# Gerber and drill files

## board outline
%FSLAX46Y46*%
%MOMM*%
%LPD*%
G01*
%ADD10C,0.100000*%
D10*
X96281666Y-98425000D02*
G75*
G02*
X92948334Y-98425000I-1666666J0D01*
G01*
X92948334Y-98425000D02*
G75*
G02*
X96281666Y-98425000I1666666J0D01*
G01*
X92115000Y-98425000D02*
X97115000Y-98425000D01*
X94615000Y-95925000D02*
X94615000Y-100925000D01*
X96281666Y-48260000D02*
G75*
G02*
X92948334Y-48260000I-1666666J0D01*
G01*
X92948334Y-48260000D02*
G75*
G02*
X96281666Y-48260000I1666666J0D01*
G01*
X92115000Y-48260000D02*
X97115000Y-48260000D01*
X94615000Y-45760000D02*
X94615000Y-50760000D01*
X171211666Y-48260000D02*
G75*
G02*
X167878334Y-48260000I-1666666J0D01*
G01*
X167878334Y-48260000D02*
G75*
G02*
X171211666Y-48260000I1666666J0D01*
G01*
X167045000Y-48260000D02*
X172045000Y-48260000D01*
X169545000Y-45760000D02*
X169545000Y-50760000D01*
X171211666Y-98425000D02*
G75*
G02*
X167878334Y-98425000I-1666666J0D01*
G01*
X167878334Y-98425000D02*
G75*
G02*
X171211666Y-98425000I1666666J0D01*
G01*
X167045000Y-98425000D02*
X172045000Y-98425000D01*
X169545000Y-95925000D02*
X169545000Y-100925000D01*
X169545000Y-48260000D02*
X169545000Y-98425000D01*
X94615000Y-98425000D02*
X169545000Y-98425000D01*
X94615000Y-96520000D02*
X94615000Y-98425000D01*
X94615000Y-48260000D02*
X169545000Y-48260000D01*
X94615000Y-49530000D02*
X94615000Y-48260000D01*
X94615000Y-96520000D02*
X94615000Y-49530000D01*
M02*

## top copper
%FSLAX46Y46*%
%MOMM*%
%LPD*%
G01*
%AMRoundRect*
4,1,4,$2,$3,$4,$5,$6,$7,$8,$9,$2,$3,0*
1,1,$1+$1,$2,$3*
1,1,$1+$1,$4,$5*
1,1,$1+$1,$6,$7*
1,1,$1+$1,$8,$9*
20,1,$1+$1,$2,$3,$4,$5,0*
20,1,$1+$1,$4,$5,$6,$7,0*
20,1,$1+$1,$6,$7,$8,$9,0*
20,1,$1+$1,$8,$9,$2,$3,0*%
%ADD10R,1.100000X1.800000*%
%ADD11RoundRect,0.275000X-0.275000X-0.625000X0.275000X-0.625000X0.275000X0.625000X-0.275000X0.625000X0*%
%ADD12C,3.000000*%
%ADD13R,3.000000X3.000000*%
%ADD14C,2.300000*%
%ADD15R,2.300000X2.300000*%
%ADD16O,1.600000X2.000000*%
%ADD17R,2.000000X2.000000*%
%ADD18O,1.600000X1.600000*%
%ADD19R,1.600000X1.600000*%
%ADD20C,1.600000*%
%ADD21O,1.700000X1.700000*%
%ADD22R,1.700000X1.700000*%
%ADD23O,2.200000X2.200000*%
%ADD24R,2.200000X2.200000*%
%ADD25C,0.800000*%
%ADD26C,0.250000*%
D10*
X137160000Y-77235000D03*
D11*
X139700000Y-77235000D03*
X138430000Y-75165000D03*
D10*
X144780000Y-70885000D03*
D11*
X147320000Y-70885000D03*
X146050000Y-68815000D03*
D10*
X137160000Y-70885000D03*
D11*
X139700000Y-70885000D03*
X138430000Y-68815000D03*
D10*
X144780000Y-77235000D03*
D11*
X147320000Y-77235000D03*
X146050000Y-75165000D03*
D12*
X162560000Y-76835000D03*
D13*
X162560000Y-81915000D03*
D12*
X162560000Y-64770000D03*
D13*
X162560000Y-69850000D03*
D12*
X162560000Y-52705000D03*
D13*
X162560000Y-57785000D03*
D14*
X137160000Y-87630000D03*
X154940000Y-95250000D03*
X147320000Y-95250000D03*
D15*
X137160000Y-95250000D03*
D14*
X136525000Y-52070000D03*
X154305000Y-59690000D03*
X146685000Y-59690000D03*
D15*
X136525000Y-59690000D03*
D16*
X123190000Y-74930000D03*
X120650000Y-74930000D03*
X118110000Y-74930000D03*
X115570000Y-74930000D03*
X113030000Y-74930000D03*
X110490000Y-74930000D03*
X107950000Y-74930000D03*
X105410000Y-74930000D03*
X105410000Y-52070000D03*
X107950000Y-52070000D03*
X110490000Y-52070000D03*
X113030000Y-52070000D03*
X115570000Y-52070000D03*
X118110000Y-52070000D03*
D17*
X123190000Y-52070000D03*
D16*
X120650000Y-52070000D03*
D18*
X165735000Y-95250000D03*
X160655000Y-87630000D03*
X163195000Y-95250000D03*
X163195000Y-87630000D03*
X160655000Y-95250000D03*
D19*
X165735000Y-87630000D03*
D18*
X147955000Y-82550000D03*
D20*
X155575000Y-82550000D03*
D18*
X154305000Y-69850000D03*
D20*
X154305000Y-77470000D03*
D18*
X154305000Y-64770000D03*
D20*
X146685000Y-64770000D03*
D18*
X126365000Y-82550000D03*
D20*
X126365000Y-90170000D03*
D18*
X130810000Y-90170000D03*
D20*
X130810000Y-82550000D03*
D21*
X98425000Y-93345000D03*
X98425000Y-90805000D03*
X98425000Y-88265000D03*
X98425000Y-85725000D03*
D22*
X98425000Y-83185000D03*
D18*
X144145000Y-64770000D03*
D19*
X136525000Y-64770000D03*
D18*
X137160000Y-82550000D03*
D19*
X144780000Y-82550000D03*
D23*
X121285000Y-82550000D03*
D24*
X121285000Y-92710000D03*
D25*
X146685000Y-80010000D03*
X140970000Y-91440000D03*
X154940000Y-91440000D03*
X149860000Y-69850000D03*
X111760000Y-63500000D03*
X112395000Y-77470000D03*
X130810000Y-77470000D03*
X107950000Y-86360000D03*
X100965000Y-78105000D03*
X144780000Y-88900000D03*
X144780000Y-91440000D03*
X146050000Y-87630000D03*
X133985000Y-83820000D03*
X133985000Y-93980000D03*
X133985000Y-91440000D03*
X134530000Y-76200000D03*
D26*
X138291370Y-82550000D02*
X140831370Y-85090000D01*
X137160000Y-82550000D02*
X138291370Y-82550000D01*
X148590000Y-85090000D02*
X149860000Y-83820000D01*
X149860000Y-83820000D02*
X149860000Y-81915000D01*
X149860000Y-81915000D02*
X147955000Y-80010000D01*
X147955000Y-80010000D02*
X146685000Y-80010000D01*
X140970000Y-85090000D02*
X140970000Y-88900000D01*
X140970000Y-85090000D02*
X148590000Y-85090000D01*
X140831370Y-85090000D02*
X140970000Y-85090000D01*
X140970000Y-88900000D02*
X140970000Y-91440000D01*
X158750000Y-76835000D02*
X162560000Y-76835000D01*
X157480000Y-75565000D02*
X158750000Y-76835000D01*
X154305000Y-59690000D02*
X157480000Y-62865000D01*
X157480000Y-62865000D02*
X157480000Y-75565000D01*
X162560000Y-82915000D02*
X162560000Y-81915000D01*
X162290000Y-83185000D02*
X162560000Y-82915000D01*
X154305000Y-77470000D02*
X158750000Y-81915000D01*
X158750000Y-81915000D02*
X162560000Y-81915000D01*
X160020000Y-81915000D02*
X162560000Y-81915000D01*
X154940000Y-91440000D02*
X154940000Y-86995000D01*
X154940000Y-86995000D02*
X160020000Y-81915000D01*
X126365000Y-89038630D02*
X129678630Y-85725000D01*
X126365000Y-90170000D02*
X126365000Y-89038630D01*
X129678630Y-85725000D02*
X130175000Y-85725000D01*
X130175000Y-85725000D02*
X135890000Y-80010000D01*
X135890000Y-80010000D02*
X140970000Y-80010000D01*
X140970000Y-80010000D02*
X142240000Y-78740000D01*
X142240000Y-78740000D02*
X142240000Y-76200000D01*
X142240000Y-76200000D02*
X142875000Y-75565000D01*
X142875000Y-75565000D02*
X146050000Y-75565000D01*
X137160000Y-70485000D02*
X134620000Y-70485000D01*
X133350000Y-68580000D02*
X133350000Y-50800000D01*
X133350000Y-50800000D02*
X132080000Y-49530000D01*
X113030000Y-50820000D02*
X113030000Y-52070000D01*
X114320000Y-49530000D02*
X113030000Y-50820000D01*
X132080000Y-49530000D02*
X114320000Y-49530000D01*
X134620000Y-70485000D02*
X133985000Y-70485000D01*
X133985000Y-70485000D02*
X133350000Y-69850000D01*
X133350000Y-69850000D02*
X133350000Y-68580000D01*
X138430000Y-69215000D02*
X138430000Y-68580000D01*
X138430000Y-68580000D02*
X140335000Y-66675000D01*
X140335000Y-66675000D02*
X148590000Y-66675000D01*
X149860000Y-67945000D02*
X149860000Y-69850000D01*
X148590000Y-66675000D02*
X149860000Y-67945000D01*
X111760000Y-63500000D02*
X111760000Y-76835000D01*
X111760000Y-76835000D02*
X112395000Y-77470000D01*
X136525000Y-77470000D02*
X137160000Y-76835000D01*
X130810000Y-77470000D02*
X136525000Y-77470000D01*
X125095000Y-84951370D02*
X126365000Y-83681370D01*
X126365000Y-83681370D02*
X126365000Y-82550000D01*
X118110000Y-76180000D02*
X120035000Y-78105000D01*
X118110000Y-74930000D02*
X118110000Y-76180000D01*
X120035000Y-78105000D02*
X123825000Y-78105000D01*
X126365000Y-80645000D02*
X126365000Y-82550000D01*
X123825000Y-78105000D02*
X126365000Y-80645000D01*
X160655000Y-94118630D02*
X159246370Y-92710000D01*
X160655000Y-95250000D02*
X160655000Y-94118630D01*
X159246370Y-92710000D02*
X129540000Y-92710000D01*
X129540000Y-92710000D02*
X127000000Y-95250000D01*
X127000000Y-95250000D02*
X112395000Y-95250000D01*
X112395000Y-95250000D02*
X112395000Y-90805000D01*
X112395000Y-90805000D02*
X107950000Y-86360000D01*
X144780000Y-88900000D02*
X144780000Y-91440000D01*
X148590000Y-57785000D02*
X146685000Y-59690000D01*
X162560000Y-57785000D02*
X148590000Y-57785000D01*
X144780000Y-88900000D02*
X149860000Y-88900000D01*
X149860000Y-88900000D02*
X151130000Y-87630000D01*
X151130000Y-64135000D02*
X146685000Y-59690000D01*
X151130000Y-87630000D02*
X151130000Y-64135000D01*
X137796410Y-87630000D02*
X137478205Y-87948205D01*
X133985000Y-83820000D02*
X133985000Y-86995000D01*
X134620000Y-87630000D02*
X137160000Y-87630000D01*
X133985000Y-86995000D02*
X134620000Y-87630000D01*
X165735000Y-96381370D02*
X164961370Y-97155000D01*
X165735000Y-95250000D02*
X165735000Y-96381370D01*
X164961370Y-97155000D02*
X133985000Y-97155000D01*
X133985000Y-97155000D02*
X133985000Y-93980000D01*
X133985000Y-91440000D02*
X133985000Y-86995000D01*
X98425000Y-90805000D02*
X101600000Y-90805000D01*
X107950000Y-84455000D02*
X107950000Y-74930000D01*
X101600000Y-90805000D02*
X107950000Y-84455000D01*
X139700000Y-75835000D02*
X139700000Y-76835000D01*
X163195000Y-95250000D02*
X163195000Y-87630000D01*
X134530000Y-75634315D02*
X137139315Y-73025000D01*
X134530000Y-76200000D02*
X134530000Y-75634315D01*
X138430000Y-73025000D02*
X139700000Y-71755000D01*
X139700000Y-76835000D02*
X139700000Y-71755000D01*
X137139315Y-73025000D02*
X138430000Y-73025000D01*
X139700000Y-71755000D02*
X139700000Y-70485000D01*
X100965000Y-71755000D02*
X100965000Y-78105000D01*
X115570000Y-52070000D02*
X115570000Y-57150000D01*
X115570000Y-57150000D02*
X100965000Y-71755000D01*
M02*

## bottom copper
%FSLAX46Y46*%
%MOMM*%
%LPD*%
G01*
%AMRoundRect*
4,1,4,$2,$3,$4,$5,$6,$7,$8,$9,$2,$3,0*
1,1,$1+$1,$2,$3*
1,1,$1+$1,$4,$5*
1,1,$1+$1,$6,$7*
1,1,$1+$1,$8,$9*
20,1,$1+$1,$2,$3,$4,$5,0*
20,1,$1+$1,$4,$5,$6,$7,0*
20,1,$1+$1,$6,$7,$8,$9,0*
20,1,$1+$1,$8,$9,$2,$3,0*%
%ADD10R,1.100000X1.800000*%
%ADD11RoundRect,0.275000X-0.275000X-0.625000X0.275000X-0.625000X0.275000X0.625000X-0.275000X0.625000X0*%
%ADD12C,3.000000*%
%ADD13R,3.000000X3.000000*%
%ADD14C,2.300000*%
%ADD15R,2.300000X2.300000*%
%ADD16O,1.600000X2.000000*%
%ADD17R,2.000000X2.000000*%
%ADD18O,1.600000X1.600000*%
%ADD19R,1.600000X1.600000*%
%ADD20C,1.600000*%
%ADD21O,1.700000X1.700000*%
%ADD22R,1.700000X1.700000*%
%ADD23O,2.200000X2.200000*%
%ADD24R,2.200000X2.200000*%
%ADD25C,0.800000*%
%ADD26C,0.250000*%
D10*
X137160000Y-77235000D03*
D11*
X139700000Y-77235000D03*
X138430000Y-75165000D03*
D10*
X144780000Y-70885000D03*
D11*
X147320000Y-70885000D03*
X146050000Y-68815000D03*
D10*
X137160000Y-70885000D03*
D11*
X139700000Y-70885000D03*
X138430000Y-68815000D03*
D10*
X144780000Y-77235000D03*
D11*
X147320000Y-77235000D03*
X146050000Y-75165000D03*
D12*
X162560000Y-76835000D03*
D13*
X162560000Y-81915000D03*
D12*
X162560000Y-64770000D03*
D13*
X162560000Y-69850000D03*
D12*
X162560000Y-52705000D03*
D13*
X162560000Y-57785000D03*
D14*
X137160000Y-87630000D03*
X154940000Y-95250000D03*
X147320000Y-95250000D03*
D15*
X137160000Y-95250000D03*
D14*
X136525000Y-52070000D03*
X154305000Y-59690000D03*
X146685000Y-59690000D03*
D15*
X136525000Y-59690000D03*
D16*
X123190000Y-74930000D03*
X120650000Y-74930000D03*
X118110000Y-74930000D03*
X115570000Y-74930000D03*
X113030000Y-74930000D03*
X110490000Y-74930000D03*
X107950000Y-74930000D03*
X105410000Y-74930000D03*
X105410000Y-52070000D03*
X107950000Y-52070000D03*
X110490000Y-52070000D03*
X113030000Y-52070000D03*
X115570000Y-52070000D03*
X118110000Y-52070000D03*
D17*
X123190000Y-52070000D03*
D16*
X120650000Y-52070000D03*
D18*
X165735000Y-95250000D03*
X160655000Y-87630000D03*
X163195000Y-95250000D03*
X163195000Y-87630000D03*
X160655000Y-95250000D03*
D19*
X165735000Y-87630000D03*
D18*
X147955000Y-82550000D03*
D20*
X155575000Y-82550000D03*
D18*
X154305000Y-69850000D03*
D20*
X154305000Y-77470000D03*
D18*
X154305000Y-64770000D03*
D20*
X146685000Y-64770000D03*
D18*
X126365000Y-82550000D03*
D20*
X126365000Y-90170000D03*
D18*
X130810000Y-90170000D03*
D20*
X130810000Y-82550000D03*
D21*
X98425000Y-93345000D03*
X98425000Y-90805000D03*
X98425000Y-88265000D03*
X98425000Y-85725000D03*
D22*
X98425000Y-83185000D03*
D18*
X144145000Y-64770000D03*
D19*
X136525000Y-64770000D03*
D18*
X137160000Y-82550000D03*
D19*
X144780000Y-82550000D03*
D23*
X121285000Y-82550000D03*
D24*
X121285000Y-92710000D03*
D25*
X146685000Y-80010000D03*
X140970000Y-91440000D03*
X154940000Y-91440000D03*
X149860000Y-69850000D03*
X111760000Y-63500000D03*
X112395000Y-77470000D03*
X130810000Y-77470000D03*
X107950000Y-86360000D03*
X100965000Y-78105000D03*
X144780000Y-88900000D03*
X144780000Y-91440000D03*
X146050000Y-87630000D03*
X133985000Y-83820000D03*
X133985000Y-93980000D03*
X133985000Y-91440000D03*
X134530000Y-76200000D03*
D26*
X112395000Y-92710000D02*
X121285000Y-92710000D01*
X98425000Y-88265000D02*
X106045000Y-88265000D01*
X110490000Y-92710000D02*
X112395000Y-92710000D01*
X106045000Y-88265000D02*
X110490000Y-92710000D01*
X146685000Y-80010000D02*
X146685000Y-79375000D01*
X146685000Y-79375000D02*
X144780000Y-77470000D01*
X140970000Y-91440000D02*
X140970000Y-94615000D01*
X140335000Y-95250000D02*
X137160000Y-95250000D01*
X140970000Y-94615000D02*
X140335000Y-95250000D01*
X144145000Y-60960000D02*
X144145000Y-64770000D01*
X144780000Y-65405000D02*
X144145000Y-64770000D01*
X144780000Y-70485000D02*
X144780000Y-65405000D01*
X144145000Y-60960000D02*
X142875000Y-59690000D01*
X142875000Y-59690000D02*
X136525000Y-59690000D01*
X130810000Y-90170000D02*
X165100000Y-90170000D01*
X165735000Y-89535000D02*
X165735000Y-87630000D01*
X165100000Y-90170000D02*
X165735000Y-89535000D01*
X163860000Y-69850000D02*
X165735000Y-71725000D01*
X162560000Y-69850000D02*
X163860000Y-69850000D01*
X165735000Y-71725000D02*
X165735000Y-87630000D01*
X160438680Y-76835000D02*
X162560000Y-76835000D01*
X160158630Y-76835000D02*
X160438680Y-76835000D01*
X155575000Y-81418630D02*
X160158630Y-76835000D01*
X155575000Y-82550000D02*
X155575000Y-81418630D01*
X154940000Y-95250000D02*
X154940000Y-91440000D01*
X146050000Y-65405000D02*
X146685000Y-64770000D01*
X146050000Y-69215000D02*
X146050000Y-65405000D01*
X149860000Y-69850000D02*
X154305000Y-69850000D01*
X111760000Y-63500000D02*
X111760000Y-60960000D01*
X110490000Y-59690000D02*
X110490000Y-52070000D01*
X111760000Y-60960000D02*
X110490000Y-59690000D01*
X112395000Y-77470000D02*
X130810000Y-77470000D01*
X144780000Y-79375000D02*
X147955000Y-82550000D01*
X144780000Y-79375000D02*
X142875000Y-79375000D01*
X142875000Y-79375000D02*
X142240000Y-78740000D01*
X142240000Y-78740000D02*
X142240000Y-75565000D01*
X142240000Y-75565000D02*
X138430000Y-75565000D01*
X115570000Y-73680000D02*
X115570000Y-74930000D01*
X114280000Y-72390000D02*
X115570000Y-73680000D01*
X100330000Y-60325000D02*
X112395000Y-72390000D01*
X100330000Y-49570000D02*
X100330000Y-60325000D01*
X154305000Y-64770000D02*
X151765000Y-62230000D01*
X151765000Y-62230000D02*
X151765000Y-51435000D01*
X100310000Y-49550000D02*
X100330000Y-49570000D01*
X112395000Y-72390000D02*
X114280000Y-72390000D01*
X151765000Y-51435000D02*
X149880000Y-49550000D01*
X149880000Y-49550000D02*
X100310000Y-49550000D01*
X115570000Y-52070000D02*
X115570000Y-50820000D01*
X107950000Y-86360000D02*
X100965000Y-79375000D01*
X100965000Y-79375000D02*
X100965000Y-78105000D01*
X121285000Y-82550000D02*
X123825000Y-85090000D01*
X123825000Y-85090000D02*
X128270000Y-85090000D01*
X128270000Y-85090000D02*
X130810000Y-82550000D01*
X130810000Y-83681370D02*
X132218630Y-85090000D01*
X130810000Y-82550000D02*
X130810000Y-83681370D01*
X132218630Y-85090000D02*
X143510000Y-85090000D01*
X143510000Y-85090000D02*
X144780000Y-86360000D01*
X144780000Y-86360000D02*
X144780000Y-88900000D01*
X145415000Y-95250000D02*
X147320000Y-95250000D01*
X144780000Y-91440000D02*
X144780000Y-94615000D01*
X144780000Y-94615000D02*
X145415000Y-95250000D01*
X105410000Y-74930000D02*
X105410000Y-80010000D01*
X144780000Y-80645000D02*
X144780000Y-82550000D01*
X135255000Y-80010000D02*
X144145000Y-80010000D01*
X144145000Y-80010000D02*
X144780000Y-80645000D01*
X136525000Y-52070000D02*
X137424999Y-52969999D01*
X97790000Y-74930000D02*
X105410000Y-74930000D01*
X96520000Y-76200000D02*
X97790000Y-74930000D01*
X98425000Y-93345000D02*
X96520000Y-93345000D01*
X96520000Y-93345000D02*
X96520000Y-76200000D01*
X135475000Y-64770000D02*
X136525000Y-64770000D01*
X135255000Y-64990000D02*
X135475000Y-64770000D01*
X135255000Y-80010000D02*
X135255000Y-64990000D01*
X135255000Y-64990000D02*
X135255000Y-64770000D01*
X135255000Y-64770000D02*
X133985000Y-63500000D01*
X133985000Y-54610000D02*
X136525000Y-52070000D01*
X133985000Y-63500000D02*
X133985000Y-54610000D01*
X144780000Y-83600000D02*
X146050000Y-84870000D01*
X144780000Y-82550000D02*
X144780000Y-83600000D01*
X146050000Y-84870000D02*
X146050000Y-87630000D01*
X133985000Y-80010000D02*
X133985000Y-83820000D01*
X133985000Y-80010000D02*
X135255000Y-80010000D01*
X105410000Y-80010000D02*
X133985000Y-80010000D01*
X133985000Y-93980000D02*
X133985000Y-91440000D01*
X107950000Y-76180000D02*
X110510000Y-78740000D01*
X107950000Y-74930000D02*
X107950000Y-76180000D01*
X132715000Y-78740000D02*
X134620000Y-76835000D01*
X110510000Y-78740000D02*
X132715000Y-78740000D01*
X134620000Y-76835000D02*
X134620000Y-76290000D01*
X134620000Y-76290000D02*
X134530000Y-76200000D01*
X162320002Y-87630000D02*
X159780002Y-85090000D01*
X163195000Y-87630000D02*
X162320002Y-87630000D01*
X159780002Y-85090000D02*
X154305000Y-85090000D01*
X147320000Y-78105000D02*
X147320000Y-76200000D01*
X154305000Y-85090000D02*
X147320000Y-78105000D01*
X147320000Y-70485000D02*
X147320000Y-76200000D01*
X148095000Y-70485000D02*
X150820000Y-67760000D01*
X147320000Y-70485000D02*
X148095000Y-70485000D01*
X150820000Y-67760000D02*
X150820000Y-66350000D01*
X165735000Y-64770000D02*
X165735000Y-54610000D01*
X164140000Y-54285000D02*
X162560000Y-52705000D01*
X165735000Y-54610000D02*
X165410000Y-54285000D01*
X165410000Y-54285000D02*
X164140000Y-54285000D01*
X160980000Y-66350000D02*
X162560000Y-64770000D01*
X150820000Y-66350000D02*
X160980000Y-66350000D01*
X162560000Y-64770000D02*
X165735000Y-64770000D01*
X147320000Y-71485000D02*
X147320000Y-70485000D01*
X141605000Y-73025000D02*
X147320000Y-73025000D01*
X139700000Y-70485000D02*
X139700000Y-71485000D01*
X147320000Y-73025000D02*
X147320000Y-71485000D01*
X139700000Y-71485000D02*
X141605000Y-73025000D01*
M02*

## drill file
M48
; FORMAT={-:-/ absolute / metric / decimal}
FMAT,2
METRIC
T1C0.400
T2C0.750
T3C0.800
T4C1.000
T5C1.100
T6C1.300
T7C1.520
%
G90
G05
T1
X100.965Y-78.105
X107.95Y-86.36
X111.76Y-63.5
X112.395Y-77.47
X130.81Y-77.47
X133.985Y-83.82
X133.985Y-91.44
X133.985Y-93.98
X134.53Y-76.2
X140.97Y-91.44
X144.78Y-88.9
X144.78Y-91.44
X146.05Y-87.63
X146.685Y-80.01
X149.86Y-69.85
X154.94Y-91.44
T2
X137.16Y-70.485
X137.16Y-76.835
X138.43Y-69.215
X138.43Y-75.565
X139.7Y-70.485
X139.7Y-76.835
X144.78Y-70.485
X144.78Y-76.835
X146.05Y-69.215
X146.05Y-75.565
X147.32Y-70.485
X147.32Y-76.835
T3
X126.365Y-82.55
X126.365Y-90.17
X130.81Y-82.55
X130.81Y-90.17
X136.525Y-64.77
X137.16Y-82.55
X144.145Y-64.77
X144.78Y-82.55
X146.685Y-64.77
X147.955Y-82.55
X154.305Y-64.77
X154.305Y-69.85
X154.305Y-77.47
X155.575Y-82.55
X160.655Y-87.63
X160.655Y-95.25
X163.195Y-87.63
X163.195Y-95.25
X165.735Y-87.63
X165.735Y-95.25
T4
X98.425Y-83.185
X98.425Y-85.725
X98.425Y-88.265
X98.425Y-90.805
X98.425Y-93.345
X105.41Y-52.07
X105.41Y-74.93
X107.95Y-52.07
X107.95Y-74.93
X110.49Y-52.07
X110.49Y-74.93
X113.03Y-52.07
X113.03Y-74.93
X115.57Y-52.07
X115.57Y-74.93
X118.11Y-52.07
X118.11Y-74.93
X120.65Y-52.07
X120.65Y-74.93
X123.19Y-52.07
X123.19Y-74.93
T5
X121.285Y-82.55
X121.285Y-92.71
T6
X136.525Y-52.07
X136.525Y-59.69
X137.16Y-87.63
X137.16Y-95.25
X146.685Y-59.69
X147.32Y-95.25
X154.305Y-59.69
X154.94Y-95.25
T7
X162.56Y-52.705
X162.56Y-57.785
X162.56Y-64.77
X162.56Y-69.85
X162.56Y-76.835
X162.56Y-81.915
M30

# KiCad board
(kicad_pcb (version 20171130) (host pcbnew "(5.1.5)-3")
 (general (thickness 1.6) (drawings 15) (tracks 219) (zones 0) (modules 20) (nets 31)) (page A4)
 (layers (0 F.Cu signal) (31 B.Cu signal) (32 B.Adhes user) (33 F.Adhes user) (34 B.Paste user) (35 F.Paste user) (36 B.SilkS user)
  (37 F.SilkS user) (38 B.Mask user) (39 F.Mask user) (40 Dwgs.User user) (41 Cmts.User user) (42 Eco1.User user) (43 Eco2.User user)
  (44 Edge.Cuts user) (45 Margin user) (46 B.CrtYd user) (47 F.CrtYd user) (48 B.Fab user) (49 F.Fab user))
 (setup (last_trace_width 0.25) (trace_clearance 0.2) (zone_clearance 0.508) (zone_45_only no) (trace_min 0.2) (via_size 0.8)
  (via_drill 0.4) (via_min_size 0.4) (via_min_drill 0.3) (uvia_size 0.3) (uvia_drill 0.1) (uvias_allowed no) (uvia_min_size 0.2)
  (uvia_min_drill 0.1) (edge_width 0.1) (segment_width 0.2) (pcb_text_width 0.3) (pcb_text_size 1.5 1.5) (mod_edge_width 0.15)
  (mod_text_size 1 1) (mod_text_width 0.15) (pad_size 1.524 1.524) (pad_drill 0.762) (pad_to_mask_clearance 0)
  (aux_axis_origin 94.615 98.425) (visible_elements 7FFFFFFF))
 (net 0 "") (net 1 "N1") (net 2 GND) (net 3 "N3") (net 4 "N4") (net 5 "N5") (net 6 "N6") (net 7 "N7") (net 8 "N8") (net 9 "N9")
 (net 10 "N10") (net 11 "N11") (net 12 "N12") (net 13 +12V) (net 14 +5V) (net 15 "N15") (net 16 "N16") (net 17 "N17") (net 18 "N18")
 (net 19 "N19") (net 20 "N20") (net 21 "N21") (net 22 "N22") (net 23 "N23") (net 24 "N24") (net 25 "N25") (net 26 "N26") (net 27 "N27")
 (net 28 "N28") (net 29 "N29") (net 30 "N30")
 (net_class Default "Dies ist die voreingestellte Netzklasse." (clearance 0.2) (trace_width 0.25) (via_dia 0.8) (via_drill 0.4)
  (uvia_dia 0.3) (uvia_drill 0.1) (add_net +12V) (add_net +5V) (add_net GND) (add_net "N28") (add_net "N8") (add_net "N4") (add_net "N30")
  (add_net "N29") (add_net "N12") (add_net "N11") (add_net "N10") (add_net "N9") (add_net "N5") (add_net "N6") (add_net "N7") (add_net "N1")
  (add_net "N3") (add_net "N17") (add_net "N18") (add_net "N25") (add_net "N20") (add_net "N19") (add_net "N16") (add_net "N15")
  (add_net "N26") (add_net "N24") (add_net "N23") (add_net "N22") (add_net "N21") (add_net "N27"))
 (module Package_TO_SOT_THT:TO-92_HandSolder (layer F.Cu) (at 137.16 76.835)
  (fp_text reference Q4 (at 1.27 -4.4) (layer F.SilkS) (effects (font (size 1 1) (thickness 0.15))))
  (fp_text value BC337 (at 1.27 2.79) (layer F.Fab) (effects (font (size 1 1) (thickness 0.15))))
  (pad 1 thru_hole rect (at 0 0) (size 1.1 1.8) (drill 0.75 (offset 0 0.4)) (layers *.Cu *.Mask) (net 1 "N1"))
  (pad 3 thru_hole roundrect (at 2.54 0) (size 1.1 1.8) (drill 0.75 (offset 0 0.4)) (layers *.Cu *.Mask) (roundrect_rratio 0.25) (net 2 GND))
  (pad 2 thru_hole roundrect (at 1.27 -1.27) (size 1.1 1.8) (drill 0.75 (offset 0 -0.4)) (layers *.Cu *.Mask) (roundrect_rratio 0.25)
   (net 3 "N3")))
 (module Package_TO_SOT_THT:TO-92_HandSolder (layer F.Cu) (at 144.78 70.485)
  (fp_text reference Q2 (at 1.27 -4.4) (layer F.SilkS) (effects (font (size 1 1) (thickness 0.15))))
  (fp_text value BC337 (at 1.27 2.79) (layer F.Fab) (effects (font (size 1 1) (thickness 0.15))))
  (pad 1 thru_hole rect (at 0 0) (size 1.1 1.8) (drill 0.75 (offset 0 0.4)) (layers *.Cu *.Mask) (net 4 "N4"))
  (pad 3 thru_hole roundrect (at 2.54 0) (size 1.1 1.8) (drill 0.75 (offset 0 0.4)) (layers *.Cu *.Mask) (roundrect_rratio 0.25) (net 2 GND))
  (pad 2 thru_hole roundrect (at 1.27 -1.27) (size 1.1 1.8) (drill 0.75 (offset 0 -0.4)) (layers *.Cu *.Mask) (roundrect_rratio 0.25)
   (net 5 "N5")))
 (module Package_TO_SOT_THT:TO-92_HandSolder (layer F.Cu) (at 137.16 70.485)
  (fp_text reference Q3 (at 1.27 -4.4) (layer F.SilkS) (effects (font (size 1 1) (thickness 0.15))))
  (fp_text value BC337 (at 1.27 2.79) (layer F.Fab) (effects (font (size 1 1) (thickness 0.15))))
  (pad 1 thru_hole rect (at 0 0) (size 1.1 1.8) (drill 0.75 (offset 0 0.4)) (layers *.Cu *.Mask) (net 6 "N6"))
  (pad 3 thru_hole roundrect (at 2.54 0) (size 1.1 1.8) (drill 0.75 (offset 0 0.4)) (layers *.Cu *.Mask) (roundrect_rratio 0.25) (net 2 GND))
  (pad 2 thru_hole roundrect (at 1.27 -1.27) (size 1.1 1.8) (drill 0.75 (offset 0 -0.4)) (layers *.Cu *.Mask) (roundrect_rratio 0.25)
   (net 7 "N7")))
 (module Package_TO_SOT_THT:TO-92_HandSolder (layer F.Cu) (at 144.78 76.835)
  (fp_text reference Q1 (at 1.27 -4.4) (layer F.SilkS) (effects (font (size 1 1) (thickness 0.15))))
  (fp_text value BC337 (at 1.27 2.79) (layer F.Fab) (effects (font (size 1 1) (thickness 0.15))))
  (pad 1 thru_hole rect (at 0 0) (size 1.1 1.8) (drill 0.75 (offset 0 0.4)) (layers *.Cu *.Mask) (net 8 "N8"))
  (pad 3 thru_hole roundrect (at 2.54 0) (size 1.1 1.8) (drill 0.75 (offset 0 0.4)) (layers *.Cu *.Mask) (roundrect_rratio 0.25) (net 2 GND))
  (pad 2 thru_hole roundrect (at 1.27 -1.27) (size 1.1 1.8) (drill 0.75 (offset 0 -0.4)) (layers *.Cu *.Mask) (roundrect_rratio 0.25)
   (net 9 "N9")))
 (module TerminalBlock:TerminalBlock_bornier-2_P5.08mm (layer F.Cu) (at 162.56 81.915 90)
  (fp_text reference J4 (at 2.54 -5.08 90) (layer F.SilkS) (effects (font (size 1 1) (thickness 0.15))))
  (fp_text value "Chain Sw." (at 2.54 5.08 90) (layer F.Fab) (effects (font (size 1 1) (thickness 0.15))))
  (pad 2 thru_hole circle (at 5.08 0 90) (size 3 3) (drill 1.52) (layers *.Cu *.Mask) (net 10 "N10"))
  (pad 1 thru_hole rect (at 0 0 90) (size 3 3) (drill 1.52) (layers *.Cu *.Mask) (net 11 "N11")))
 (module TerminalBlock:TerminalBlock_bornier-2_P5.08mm (layer F.Cu) (at 162.56 69.85 90)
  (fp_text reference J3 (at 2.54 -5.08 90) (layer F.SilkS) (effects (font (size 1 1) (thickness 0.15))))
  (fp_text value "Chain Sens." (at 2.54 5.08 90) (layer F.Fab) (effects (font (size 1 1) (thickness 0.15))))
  (pad 2 thru_hole circle (at 5.08 0 90) (size 3 3) (drill 1.52) (layers *.Cu *.Mask) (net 2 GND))
  (pad 1 thru_hole rect (at 0 0 90) (size 3 3) (drill 1.52) (layers *.Cu *.Mask) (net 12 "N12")))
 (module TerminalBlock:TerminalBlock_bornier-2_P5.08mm (layer F.Cu) (at 162.56 57.785 90)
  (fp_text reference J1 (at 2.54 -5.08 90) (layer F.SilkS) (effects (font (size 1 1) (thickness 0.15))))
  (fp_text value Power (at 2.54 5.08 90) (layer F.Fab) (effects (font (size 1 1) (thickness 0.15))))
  (pad 2 thru_hole circle (at 5.08 0 90) (size 3 3) (drill 1.52) (layers *.Cu *.Mask) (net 2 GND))
  (pad 1 thru_hole rect (at 0 0 90) (size 3 3) (drill 1.52) (layers *.Cu *.Mask) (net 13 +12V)))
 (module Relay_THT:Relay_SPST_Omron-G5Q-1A (layer F.Cu) (at 137.16 95.25)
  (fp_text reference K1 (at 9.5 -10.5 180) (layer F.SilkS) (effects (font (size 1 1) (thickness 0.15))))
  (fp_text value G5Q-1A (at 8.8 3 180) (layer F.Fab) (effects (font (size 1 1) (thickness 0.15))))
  (pad 5 thru_hole circle (at 0 -7.62 180) (size 2.3 2.3) (drill 1.3) (layers *.Cu *.Mask) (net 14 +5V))
  (pad 3 thru_hole circle (at 17.78 0 180) (size 2.3 2.3) (drill 1.3) (layers *.Cu *.Mask) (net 11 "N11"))
  (pad 2 thru_hole circle (at 10.16 0 180) (size 2.3 2.3) (drill 1.3) (layers *.Cu *.Mask) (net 13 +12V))
  (pad 1 thru_hole rect (at 0 0 180) (size 2.3 2.3) (drill 1.3) (layers *.Cu *.Mask) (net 8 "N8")))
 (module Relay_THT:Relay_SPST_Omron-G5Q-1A (layer F.Cu) (at 136.525 59.69)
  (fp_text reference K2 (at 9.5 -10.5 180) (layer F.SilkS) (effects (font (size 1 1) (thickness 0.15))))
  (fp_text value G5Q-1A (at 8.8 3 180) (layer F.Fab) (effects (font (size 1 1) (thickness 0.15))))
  (pad 5 thru_hole circle (at 0 -7.62 180) (size 2.3 2.3) (drill 1.3) (layers *.Cu *.Mask) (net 14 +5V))
  (pad 3 thru_hole circle (at 17.78 0 180) (size 2.3 2.3) (drill 1.3) (layers *.Cu *.Mask) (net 10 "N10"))
  (pad 2 thru_hole circle (at 10.16 0 180) (size 2.3 2.3) (drill 1.3) (layers *.Cu *.Mask) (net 13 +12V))
  (pad 1 thru_hole rect (at 0 0 180) (size 2.3 2.3) (drill 1.3) (layers *.Cu *.Mask) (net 4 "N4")))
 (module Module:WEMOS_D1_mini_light (layer F.Cu) (at 123.19 52.07 270)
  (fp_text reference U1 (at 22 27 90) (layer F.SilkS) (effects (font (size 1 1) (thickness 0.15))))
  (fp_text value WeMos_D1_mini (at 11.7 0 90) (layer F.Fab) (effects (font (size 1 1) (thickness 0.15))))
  (pad 16 thru_hole oval (at 22.86 0 270) (size 2 1.6) (drill 1) (layers *.Cu *.Mask) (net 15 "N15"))
  (pad 15 thru_hole oval (at 22.86 2.54 270) (size 2 1.6) (drill 1) (layers *.Cu *.Mask) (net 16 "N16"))
  (pad 14 thru_hole oval (at 22.86 5.08 270) (size 2 1.6) (drill 1) (layers *.Cu *.Mask) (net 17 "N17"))
  (pad 13 thru_hole oval (at 22.86 7.62 270) (size 2 1.6) (drill 1) (layers *.Cu *.Mask) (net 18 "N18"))
  (pad 12 thru_hole oval (at 22.86 10.16 270) (size 2 1.6) (drill 1) (layers *.Cu *.Mask) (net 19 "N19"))
  (pad 11 thru_hole oval (at 22.86 12.7 270) (size 2 1.6) (drill 1) (layers *.Cu *.Mask) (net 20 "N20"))
  (pad 10 thru_hole oval (at 22.86 15.24 270) (size 2 1.6) (drill 1) (layers *.Cu *.Mask) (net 2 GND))
  (pad 9 thru_hole oval (at 22.86 17.78 270) (size 2 1.6) (drill 1) (layers *.Cu *.Mask) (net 14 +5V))
  (pad 8 thru_hole oval (at 0 17.78 270) (size 2 1.6) (drill 1) (layers *.Cu *.Mask) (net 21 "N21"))
  (pad 7 thru_hole oval (at 0 15.24 270) (size 2 1.6) (drill 1) (layers *.Cu *.Mask) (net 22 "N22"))
  (pad 6 thru_hole oval (at 0 12.7 270) (size 2 1.6) (drill 1) (layers *.Cu *.Mask) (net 1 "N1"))
  (pad 5 thru_hole oval (at 0 10.16 270) (size 2 1.6) (drill 1) (layers *.Cu *.Mask) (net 6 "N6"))
  (pad 4 thru_hole oval (at 0 7.62 270) (size 2 1.6) (drill 1) (layers *.Cu *.Mask) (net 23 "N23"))
  (pad 3 thru_hole oval (at 0 5.08 270) (size 2 1.6) (drill 1) (layers *.Cu *.Mask) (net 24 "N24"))
  (pad 1 thru_hole rect (at 0 0 270) (size 2 2) (drill 1) (layers *.Cu *.Mask) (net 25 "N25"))
  (pad 2 thru_hole oval (at 0 2.54 270) (size 2 1.6) (drill 1) (layers *.Cu *.Mask) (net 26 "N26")))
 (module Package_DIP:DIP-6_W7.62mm (layer F.Cu) (at 165.735 87.63 270)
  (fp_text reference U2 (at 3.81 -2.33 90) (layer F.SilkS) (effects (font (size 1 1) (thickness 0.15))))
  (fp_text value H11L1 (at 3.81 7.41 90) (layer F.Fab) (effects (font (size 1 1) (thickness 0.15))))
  (pad 6 thru_hole oval (at 7.62 0 270) (size 1.6 1.6) (drill 0.8) (layers *.Cu *.Mask) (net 14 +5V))
  (pad 3 thru_hole oval (at 0 5.08 270) (size 1.6 1.6) (drill 0.8) (layers *.Cu *.Mask) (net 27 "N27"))
  (pad 5 thru_hole oval (at 7.62 2.54 270) (size 1.6 1.6) (drill 0.8) (layers *.Cu *.Mask) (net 2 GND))
  (pad 2 thru_hole oval (at 0 2.54 270) (size 1.6 1.6) (drill 0.8) (layers *.Cu *.Mask) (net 2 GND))
  (pad 4 thru_hole oval (at 7.62 5.08 270) (size 1.6 1.6) (drill 0.8) (layers *.Cu *.Mask) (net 23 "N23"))
  (pad 1 thru_hole rect (at 0 0 270) (size 1.6 1.6) (drill 0.8) (layers *.Cu *.Mask) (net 12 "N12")))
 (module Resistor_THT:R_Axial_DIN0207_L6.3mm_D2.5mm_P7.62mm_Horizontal (layer F.Cu) (at 155.575 82.55 180)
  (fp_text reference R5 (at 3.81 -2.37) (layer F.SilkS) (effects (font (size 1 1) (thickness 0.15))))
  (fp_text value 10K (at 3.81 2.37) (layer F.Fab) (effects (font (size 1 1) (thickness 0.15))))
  (pad 2 thru_hole oval (at 7.62 0 180) (size 1.6 1.6) (drill 0.8) (layers *.Cu *.Mask) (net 3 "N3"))
  (pad 1 thru_hole circle (at 0 0 180) (size 1.6 1.6) (drill 0.8) (layers *.Cu *.Mask) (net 10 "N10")))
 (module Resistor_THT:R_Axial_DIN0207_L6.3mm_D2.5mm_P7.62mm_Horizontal (layer F.Cu) (at 154.305 77.47 90)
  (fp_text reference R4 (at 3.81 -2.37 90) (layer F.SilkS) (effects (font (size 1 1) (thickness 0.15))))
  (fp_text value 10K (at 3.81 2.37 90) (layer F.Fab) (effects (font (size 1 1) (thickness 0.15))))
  (pad 2 thru_hole oval (at 7.62 0 90) (size 1.6 1.6) (drill 0.8) (layers *.Cu *.Mask) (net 7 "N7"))
  (pad 1 thru_hole circle (at 0 0 90) (size 1.6 1.6) (drill 0.8) (layers *.Cu *.Mask) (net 11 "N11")))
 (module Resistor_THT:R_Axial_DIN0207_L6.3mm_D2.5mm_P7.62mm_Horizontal (layer F.Cu) (at 146.685 64.77)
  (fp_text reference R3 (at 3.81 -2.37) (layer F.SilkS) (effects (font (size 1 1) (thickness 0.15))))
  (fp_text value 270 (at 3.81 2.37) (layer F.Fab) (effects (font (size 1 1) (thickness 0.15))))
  (pad 2 thru_hole oval (at 7.62 0) (size 1.6 1.6) (drill 0.8) (layers *.Cu *.Mask) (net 18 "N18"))
  (pad 1 thru_hole circle (at 0 0) (size 1.6 1.6) (drill 0.8) (layers *.Cu *.Mask) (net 5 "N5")))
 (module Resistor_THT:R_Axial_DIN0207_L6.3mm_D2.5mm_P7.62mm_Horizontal (layer F.Cu) (at 126.365 90.17 90)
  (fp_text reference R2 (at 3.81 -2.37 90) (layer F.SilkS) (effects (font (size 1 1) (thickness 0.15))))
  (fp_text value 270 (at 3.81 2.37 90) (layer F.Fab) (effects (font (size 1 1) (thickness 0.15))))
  (pad 2 thru_hole oval (at 7.62 0 90) (size 1.6 1.6) (drill 0.8) (layers *.Cu *.Mask) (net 17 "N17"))
  (pad 1 thru_hole circle (at 0 0 90) (size 1.6 1.6) (drill 0.8) (layers *.Cu *.Mask) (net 9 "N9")))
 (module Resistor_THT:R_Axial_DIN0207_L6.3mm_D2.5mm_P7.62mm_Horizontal (layer F.Cu) (at 130.81 82.55 270)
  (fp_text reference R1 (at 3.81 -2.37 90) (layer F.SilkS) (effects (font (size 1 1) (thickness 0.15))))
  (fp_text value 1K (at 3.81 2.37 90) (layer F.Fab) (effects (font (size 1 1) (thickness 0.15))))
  (pad 2 thru_hole oval (at 7.62 0 270) (size 1.6 1.6) (drill 0.8) (layers *.Cu *.Mask) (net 12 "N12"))
  (pad 1 thru_hole circle (at 0 0 270) (size 1.6 1.6) (drill 0.8) (layers *.Cu *.Mask) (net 13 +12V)))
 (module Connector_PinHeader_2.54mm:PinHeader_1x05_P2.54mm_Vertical (layer F.Cu) (at 98.425 83.185)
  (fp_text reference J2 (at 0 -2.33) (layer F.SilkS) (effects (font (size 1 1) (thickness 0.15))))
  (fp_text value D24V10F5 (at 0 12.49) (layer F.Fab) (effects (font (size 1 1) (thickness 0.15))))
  (pad 5 thru_hole oval (at 0 10.16) (size 1.7 1.7) (drill 1) (layers *.Cu *.Mask) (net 14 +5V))
  (pad 4 thru_hole oval (at 0 7.62) (size 1.7 1.7) (drill 1) (layers *.Cu *.Mask) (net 2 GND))
  (pad 3 thru_hole oval (at 0 5.08) (size 1.7 1.7) (drill 1) (layers *.Cu *.Mask) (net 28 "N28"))
  (pad 2 thru_hole oval (at 0 2.54) (size 1.7 1.7) (drill 1) (layers *.Cu *.Mask) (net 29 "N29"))
  (pad 1 thru_hole rect (at 0 0) (size 1.7 1.7) (drill 1) (layers *.Cu *.Mask) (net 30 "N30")))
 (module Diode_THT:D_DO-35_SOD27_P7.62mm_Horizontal (layer F.Cu) (at 136.525 64.77)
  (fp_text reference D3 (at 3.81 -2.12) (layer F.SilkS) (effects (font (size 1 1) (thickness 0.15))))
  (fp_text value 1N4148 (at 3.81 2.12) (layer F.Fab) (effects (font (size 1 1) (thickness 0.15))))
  (pad 2 thru_hole oval (at 7.62 0) (size 1.6 1.6) (drill 0.8) (layers *.Cu *.Mask) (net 4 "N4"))
  (pad 1 thru_hole rect (at 0 0) (size 1.6 1.6) (drill 0.8) (layers *.Cu *.Mask) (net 14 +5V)))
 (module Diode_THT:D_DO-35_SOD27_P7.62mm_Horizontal (layer F.Cu) (at 144.78 82.55 180)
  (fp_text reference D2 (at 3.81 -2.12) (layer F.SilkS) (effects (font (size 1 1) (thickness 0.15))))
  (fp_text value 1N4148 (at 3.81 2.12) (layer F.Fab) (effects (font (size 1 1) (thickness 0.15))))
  (pad 2 thru_hole oval (at 7.62 0 180) (size 1.6 1.6) (drill 0.8) (layers *.Cu *.Mask) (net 8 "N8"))
  (pad 1 thru_hole rect (at 0 0 180) (size 1.6 1.6) (drill 0.8) (layers *.Cu *.Mask) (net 14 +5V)))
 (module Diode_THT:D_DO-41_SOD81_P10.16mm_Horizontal (layer F.Cu) (at 121.285 92.71 90)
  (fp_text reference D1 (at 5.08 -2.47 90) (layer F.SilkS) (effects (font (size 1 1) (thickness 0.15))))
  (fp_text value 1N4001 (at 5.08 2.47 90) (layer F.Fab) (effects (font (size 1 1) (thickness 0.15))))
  (pad 2 thru_hole oval (at 10.16 0 90) (size 2.2 2.2) (drill 1.1) (layers *.Cu *.Mask) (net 13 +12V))
  (pad 1 thru_hole rect (at 0 0 90) (size 2.2 2.2) (drill 1.1) (layers *.Cu *.Mask) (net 28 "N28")))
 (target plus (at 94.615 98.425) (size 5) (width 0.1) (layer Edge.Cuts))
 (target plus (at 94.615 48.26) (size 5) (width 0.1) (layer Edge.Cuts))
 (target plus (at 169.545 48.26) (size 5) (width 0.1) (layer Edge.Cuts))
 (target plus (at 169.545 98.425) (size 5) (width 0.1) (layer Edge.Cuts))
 (gr_line (start 169.545 48.26) (end 169.545 98.425) (layer Edge.Cuts) (width 0.1))
 (gr_line (start 94.615 98.425) (end 169.545 98.425) (layer Edge.Cuts) (width 0.1))
 (gr_line (start 94.615 96.52) (end 94.615 98.425) (layer Edge.Cuts) (width 0.1))
 (gr_line (start 94.615 48.26) (end 169.545 48.26) (layer Edge.Cuts) (width 0.1))
 (gr_line (start 94.615 49.53) (end 94.615 48.26) (layer Edge.Cuts) (width 0.1))
 (gr_line (start 94.615 96.52) (end 94.615 49.53) (layer Edge.Cuts) (width 0.1))
 (segment (start 112.395 92.71) (end 121.285 92.71) (width 0.25) (layer B.Cu) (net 28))
 (segment (start 98.425 88.265) (end 106.045 88.265) (width 0.25) (layer B.Cu) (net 28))
 (segment (start 110.49 92.71) (end 112.395 92.71) (width 0.25) (layer B.Cu) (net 28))
 (segment (start 106.045 88.265) (end 110.49 92.71) (width 0.25) (layer B.Cu) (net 28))
 (segment (start 138.29137 82.55) (end 140.83137 85.09) (width 0.25) (layer F.Cu) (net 8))
 (segment (start 137.16 82.55) (end 138.29137 82.55) (width 0.25) (layer F.Cu) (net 8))
 (segment (start 148.59 85.09) (end 149.86 83.82) (width 0.25) (layer F.Cu) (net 8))
 (segment (start 149.86 83.82) (end 149.86 81.915) (width 0.25) (layer F.Cu) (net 8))
 (segment (start 149.86 81.915) (end 147.955 80.01) (width 0.25) (layer F.Cu) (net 8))
 (via (at 146.685 80.01) (size 0.8) (drill 0.4) (layers F.Cu B.Cu) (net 8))
 (segment (start 147.955 80.01) (end 146.685 80.01) (width 0.25) (layer F.Cu) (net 8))
 (segment (start 146.685 80.01) (end 146.685 79.375) (width 0.25) (layer B.Cu) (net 8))
 (segment (start 146.685 79.375) (end 144.78 77.47) (width 0.25) (layer B.Cu) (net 8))
 (segment (start 140.97 85.09) (end 140.97 88.9) (width 0.25) (layer F.Cu) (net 8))
 (segment (start 140.97 85.09) (end 148.59 85.09) (width 0.25) (layer F.Cu) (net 8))
 (segment (start 140.83137 85.09) (end 140.97 85.09) (width 0.25) (layer F.Cu) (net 8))
 (segment (start 140.97 88.9) (end 140.97 91.44) (width 0.25) (layer F.Cu) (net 8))
 (via (at 140.97 91.44) (size 0.8) (drill 0.4) (layers F.Cu B.Cu) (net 8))
 (segment (start 140.97 91.44) (end 140.97 94.615) (width 0.25) (layer B.Cu) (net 8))
 (segment (start 140.335 95.25) (end 137.16 95.25) (width 0.25) (layer B.Cu) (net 8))
 (segment (start 140.97 94.615) (end 140.335 95.25) (width 0.25) (layer B.Cu) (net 8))
 (segment (start 144.145 60.96) (end 144.145 64.77) (width 0.25) (layer B.Cu) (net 4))
 (segment (start 144.78 65.405) (end 144.145 64.77) (width 0.25) (layer B.Cu) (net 4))
 (segment (start 144.78 70.485) (end 144.78 65.405) (width 0.25) (layer B.Cu) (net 4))
 (segment (start 144.145 60.96) (end 142.875 59.69) (width 0.25) (layer B.Cu) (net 4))
 (segment (start 142.875 59.69) (end 136.525 59.69) (width 0.25) (layer B.Cu) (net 4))
 (segment (start 130.81 90.17) (end 165.1 90.17) (width 0.25) (layer B.Cu) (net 12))
 (segment (start 165.735 89.535) (end 165.735 87.63) (width 0.25) (layer B.Cu) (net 12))
 (segment (start 165.1 90.17) (end 165.735 89.535) (width 0.25) (layer B.Cu) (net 12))
 (segment (start 163.86 69.85) (end 165.735 71.725) (width 0.25) (layer B.Cu) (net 12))
 (segment (start 162.56 69.85) (end 163.86 69.85) (width 0.25) (layer B.Cu) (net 12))
 (segment (start 165.735 71.725) (end 165.735 87.63) (width 0.25) (layer B.Cu) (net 12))
 (segment (start 158.75 76.835) (end 162.56 76.835) (width 0.25) (layer F.Cu) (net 10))
 (segment (start 157.48 75.565) (end 158.75 76.835) (width 0.25) (layer F.Cu) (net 10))
 (segment (start 154.305 59.69) (end 157.48 62.865) (width 0.25) (layer F.Cu) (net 10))
 (segment (start 157.48 62.865) (end 157.48 75.565) (width 0.25) (layer F.Cu) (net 10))
 (segment (start 160.43868 76.835) (end 162.56 76.835) (width 0.25) (layer B.Cu) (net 10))
 (segment (start 160.15863 76.835) (end 160.43868 76.835) (width 0.25) (layer B.Cu) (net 10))
 (segment (start 155.575 81.41863) (end 160.15863 76.835) (width 0.25) (layer B.Cu) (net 10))
 (segment (start 155.575 82.55) (end 155.575 81.41863) (width 0.25) (layer B.Cu) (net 10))
 (segment (start 154.94 95.25) (end 154.94 91.44) (width 0.25) (layer B.Cu) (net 11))
 (via (at 154.94 91.44) (size 0.8) (drill 0.4) (layers F.Cu B.Cu) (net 11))
 (segment (start 162.56 82.915) (end 162.56 81.915) (width 0.25) (layer F.Cu) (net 11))
 (segment (start 162.29 83.185) (end 162.56 82.915) (width 0.25) (layer F.Cu) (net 11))
 (segment (start 154.305 77.47) (end 158.75 81.915) (width 0.25) (layer F.Cu) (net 11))
 (segment (start 158.75 81.915) (end 162.56 81.915) (width 0.25) (layer F.Cu) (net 11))
 (segment (start 160.02 81.915) (end 162.56 81.915) (width 0.25) (layer F.Cu) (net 11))
 (segment (start 154.94 91.44) (end 154.94 86.995) (width 0.25) (layer F.Cu) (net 11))
 (segment (start 154.94 86.995) (end 160.02 81.915) (width 0.25) (layer F.Cu) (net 11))
 (segment (start 126.365 89.03863) (end 129.67863 85.725) (width 0.25) (layer F.Cu) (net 9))
 (segment (start 126.365 90.17) (end 126.365 89.03863) (width 0.25) (layer F.Cu) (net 9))
 (segment (start 129.67863 85.725) (end 130.175 85.725) (width 0.25) (layer F.Cu) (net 9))
 (segment (start 130.175 85.725) (end 135.89 80.01) (width 0.25) (layer F.Cu) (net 9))
 (segment (start 135.89 80.01) (end 140.97 80.01) (width 0.25) (layer F.Cu) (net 9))
 (segment (start 140.97 80.01) (end 142.24 78.74) (width 0.25) (layer F.Cu) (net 9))
 (segment (start 142.24 78.74) (end 142.24 76.2) (width 0.25) (layer F.Cu) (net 9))
 (segment (start 142.24 76.2) (end 142.875 75.565) (width 0.25) (layer F.Cu) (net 9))
 (segment (start 142.875 75.565) (end 146.05 75.565) (width 0.25) (layer F.Cu) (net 9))
 (segment (start 146.05 65.405) (end 146.685 64.77) (width 0.25) (layer B.Cu) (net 5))
 (segment (start 146.05 69.215) (end 146.05 65.405) (width 0.25) (layer B.Cu) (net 5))
 (segment (start 137.16 70.485) (end 134.62 70.485) (width 0.25) (layer F.Cu) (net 6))
 (segment (start 133.35 68.58) (end 133.35 50.8) (width 0.25) (layer F.Cu) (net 6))
 (segment (start 133.35 50.8) (end 132.08 49.53) (width 0.25) (layer F.Cu) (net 6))
 (segment (start 113.03 50.82) (end 113.03 52.07) (width 0.25) (layer F.Cu) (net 6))
 (segment (start 114.32 49.53) (end 113.03 50.82) (width 0.25) (layer F.Cu) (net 6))
 (segment (start 132.08 49.53) (end 114.32 49.53) (width 0.25) (layer F.Cu) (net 6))
 (segment (start 134.62 70.485) (end 133.985 70.485) (width 0.25) (layer F.Cu) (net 6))
 (segment (start 133.985 70.485) (end 133.35 69.85) (width 0.25) (layer F.Cu) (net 6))
 (segment (start 133.35 69.85) (end 133.35 68.58) (width 0.25) (layer F.Cu) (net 6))
 (via (at 149.86 69.85) (size 0.8) (drill 0.4) (layers F.Cu B.Cu) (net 7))
 (segment (start 149.86 69.85) (end 154.305 69.85) (width 0.25) (layer B.Cu) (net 7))
 (segment (start 138.43 69.215) (end 138.43 68.58) (width 0.25) (layer F.Cu) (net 7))
 (segment (start 138.43 68.58) (end 140.335 66.675) (width 0.25) (layer F.Cu) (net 7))
 (segment (start 140.335 66.675) (end 148.59 66.675) (width 0.25) (layer F.Cu) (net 7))
 (segment (start 149.86 67.945) (end 149.86 69.85) (width 0.25) (layer F.Cu) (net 7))
 (segment (start 148.59 66.675) (end 149.86 67.945) (width 0.25) (layer F.Cu) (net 7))
 (via (at 111.76 63.5) (size 0.8) (drill 0.4) (layers F.Cu B.Cu) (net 1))
 (segment (start 111.76 63.5) (end 111.76 60.96) (width 0.25) (layer B.Cu) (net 1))
 (segment (start 110.49 59.69) (end 110.49 52.07) (width 0.25) (layer B.Cu) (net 1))
 (segment (start 111.76 60.96) (end 110.49 59.69) (width 0.25) (layer B.Cu) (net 1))
 (segment (start 111.76 63.5) (end 111.76 76.835) (width 0.25) (layer F.Cu) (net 1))
 (segment (start 111.76 76.835) (end 112.395 77.47) (width 0.25) (layer F.Cu) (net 1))
 (via (at 112.395 77.47) (size 0.8) (drill 0.4) (layers F.Cu B.Cu) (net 1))
 (via (at 130.81 77.47) (size 0.8) (drill 0.4) (layers F.Cu B.Cu) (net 1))
 (segment (start 112.395 77.47) (end 130.81 77.47) (width 0.25) (layer B.Cu) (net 1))
 (segment (start 136.525 77.47) (end 137.16 76.835) (width 0.25) (layer F.Cu) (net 1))
 (segment (start 130.81 77.47) (end 136.525 77.47) (width 0.25) (layer F.Cu) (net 1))
 (segment (start 144.78 79.375) (end 147.955 82.55) (width 0.25) (layer B.Cu) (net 3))
 (segment (start 144.78 79.375) (end 142.875 79.375) (width 0.25) (layer B.Cu) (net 3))
 (segment (start 142.875 79.375) (end 142.24 78.74) (width 0.25) (layer B.Cu) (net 3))
 (segment (start 142.24 78.74) (end 142.24 75.565) (width 0.25) (layer B.Cu) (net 3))
 (segment (start 142.24 75.565) (end 138.43 75.565) (width 0.25) (layer B.Cu) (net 3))
 (segment (start 125.095 84.95137) (end 126.365 83.68137) (width 0.25) (layer F.Cu) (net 17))
 (segment (start 126.365 83.68137) (end 126.365 82.55) (width 0.25) (layer F.Cu) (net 17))
 (segment (start 118.11 76.18) (end 120.035 78.105) (width 0.25) (layer F.Cu) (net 17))
 (segment (start 118.11 74.93) (end 118.11 76.18) (width 0.25) (layer F.Cu) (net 17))
 (segment (start 120.035 78.105) (end 123.825 78.105) (width 0.25) (layer F.Cu) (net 17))
 (segment (start 126.365 80.645) (end 126.365 82.55) (width 0.25) (layer F.Cu) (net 17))
 (segment (start 123.825 78.105) (end 126.365 80.645) (width 0.25) (layer F.Cu) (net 17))
 (segment (start 115.57 73.68) (end 115.57 74.93) (width 0.25) (layer B.Cu) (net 18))
 (segment (start 114.28 72.39) (end 115.57 73.68) (width 0.25) (layer B.Cu) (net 18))
 (segment (start 100.33 60.325) (end 112.395 72.39) (width 0.25) (layer B.Cu) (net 18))
 (segment (start 100.33 49.57) (end 100.33 60.325) (width 0.25) (layer B.Cu) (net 18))
 (segment (start 154.305 64.77) (end 151.765 62.23) (width 0.25) (layer B.Cu) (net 18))
 (segment (start 151.765 62.23) (end 151.765 51.435) (width 0.25) (layer B.Cu) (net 18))
 (segment (start 100.31 49.55) (end 100.33 49.57) (width 0.25) (layer B.Cu) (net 18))
 (segment (start 112.395 72.39) (end 114.28 72.39) (width 0.25) (layer B.Cu) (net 18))
 (segment (start 151.765 51.435) (end 149.88 49.55) (width 0.25) (layer B.Cu) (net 18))
 (segment (start 149.88 49.55) (end 100.31 49.55) (width 0.25) (layer B.Cu) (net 18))
 (segment (start 115.57 52.07) (end 115.57 50.82) (width 0.25) (layer B.Cu) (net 23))
 (segment (start 160.655 94.11863) (end 159.24637 92.71) (width 0.25) (layer F.Cu) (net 23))
 (segment (start 160.655 95.25) (end 160.655 94.11863) (width 0.25) (layer F.Cu) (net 23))
 (segment (start 159.24637 92.71) (end 129.54 92.71) (width 0.25) (layer F.Cu) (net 23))
 (segment (start 129.54 92.71) (end 127 95.25) (width 0.25) (layer F.Cu) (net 23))
 (segment (start 127 95.25) (end 112.395 95.25) (width 0.25) (layer F.Cu) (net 23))
 (segment (start 112.395 95.25) (end 112.395 90.805) (width 0.25) (layer F.Cu) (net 23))
 (via (at 107.95 86.36) (size 0.8) (drill 0.4) (layers F.Cu B.Cu) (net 23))
 (segment (start 112.395 90.805) (end 107.95 86.36) (width 0.25) (layer F.Cu) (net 23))
 (segment (start 107.95 86.36) (end 100.965 79.375) (width 0.25) (layer B.Cu) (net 23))
 (via (at 100.965 78.105) (size 0.8) (drill 0.4) (layers F.Cu B.Cu) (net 23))
 (segment (start 100.965 79.375) (end 100.965 78.105) (width 0.25) (layer B.Cu) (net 23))
 (segment (start 121.285 82.55) (end 123.825 85.09) (width 0.25) (layer B.Cu) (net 13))
 (segment (start 123.825 85.09) (end 128.27 85.09) (width 0.25) (layer B.Cu) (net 13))
 (segment (start 128.27 85.09) (end 130.81 82.55) (width 0.25) (layer B.Cu) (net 13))
 (segment (start 130.81 83.68137) (end 132.21863 85.09) (width 0.25) (layer B.Cu) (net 13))
 (segment (start 130.81 82.55) (end 130.81 83.68137) (width 0.25) (layer B.Cu) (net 13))
 (segment (start 132.21863 85.09) (end 143.51 85.09) (width 0.25) (layer B.Cu) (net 13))
 (segment (start 143.51 85.09) (end 144.78 86.36) (width 0.25) (layer B.Cu) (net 13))
 (via (at 144.78 88.9) (size 0.8) (drill 0.4) (layers F.Cu B.Cu) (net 13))
 (segment (start 144.78 86.36) (end 144.78 88.9) (width 0.25) (layer B.Cu) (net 13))
 (segment (start 144.78 88.9) (end 144.78 91.44) (width 0.25) (layer F.Cu) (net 13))
 (via (at 144.78 91.44) (size 0.8) (drill 0.4) (layers F.Cu B.Cu) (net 13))
 (segment (start 145.415 95.25) (end 147.32 95.25) (width 0.25) (layer B.Cu) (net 13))
 (segment (start 144.78 91.44) (end 144.78 94.615) (width 0.25) (layer B.Cu) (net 13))
 (segment (start 144.78 94.615) (end 145.415 95.25) (width 0.25) (layer B.Cu) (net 13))
 (segment (start 148.59 57.785) (end 146.685 59.69) (width 0.25) (layer F.Cu) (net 13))
 (segment (start 162.56 57.785) (end 148.59 57.785) (width 0.25) (layer F.Cu) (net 13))
 (segment (start 144.78 88.9) (end 149.86 88.9) (width 0.25) (layer F.Cu) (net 13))
 (segment (start 149.86 88.9) (end 151.13 87.63) (width 0.25) (layer F.Cu) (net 13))
 (segment (start 151.13 64.135) (end 146.685 59.69) (width 0.25) (layer F.Cu) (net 13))
 (segment (start 151.13 87.63) (end 151.13 64.135) (width 0.25) (layer F.Cu) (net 13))
 (segment (start 105.41 74.93) (end 105.41 80.01) (width 0.25) (layer B.Cu) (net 14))
 (segment (start 144.78 80.645) (end 144.78 82.55) (width 0.25) (layer B.Cu) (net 14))
 (segment (start 135.255 80.01) (end 144.145 80.01) (width 0.25) (layer B.Cu) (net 14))
 (segment (start 144.145 80.01) (end 144.78 80.645) (width 0.25) (layer B.Cu) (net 14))
 (segment (start 136.525 52.07) (end 137.424999 52.969999) (width 0.25) (layer B.Cu) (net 14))
 (segment (start 97.79 74.93) (end 105.41 74.93) (width 0.25) (layer B.Cu) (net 14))
 (segment (start 96.52 76.2) (end 97.79 74.93) (width 0.25) (layer B.Cu) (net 14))
 (segment (start 98.425 93.345) (end 96.52 93.345) (width 0.25) (layer B.Cu) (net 14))
 (segment (start 96.52 93.345) (end 96.52 76.2) (width 0.25) (layer B.Cu) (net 14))
 (segment (start 135.475 64.77) (end 136.525 64.77) (width 0.25) (layer B.Cu) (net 14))
 (segment (start 135.255 64.99) (end 135.475 64.77) (width 0.25) (layer B.Cu) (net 14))
 (segment (start 135.255 80.01) (end 135.255 64.99) (width 0.25) (layer B.Cu) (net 14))
 (segment (start 135.255 64.99) (end 135.255 64.77) (width 0.25) (layer B.Cu) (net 14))
 (segment (start 135.255 64.77) (end 133.985 63.5) (width 0.25) (layer B.Cu) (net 14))
 (segment (start 133.985 54.61) (end 136.525 52.07) (width 0.25) (layer B.Cu) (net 14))
 (segment (start 133.985 63.5) (end 133.985 54.61) (width 0.25) (layer B.Cu) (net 14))
 (segment (start 144.78 83.6) (end 146.05 84.87) (width 0.25) (layer B.Cu) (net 14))
 (segment (start 144.78 82.55) (end 144.78 83.6) (width 0.25) (layer B.Cu) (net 14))
 (via (at 146.05 87.63) (size 0.8) (drill 0.4) (layers F.Cu B.Cu) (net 14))
 (segment (start 146.05 84.87) (end 146.05 87.63) (width 0.25) (layer B.Cu) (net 14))
 (segment (start 137.79641 87.63) (end 137.478205 87.948205) (width 0.25) (layer F.Cu) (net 14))
 (segment (start 133.985 80.01) (end 133.985 83.82) (width 0.25) (layer B.Cu) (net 14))
 (segment (start 133.985 80.01) (end 135.255 80.01) (width 0.25) (layer B.Cu) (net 14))
 (segment (start 105.41 80.01) (end 133.985 80.01) (width 0.25) (layer B.Cu) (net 14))
 (via (at 133.985 83.82) (size 0.8) (drill 0.4) (layers F.Cu B.Cu) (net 14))
 (segment (start 133.985 83.82) (end 133.985 86.995) (width 0.25) (layer F.Cu) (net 14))
 (segment (start 134.62 87.63) (end 137.16 87.63) (width 0.25) (layer F.Cu) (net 14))
 (segment (start 133.985 86.995) (end 134.62 87.63) (width 0.25) (layer F.Cu) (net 14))
 (segment (start 165.735 96.38137) (end 164.96137 97.155) (width 0.25) (layer F.Cu) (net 14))
 (segment (start 165.735 95.25) (end 165.735 96.38137) (width 0.25) (layer F.Cu) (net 14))
 (segment (start 164.96137 97.155) (end 133.985 97.155) (width 0.25) (layer F.Cu) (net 14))
 (segment (start 133.985 97.155) (end 133.985 93.98) (width 0.25) (layer F.Cu) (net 14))
 (via (at 133.985 93.98) (size 0.8) (drill 0.4) (layers F.Cu B.Cu) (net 14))
 (segment (start 133.985 93.98) (end 133.985 91.44) (width 0.25) (layer B.Cu) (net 14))
 (via (at 133.985 91.44) (size 0.8) (drill 0.4) (layers F.Cu B.Cu) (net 14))
 (segment (start 133.985 91.44) (end 133.985 86.995) (width 0.25) (layer F.Cu) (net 14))
 (segment (start 98.425 90.805) (end 101.6 90.805) (width 0.25) (layer F.Cu) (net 2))
 (segment (start 107.95 84.455) (end 107.95 74.93) (width 0.25) (layer F.Cu) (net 2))
 (segment (start 101.6 90.805) (end 107.95 84.455) (width 0.25) (layer F.Cu) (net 2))
 (segment (start 107.95 76.18) (end 110.51 78.74) (width 0.25) (layer B.Cu) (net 2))
 (segment (start 107.95 74.93) (end 107.95 76.18) (width 0.25) (layer B.Cu) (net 2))
 (segment (start 132.715 78.74) (end 134.62 76.835) (width 0.25) (layer B.Cu) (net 2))
 (segment (start 110.51 78.74) (end 132.715 78.74) (width 0.25) (layer B.Cu) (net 2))
 (segment (start 134.62 76.835) (end 134.62 76.29) (width 0.25) (layer B.Cu) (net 2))
 (via (at 134.53 76.2) (size 0.8) (drill 0.4) (layers F.Cu B.Cu) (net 2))
 (segment (start 134.62 76.29) (end 134.53 76.2) (width 0.25) (layer B.Cu) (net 2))
 (segment (start 139.7 75.835) (end 139.7 76.835) (width 0.25) (layer F.Cu) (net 2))
 (segment (start 163.195 95.25) (end 163.195 87.63) (width 0.25) (layer F.Cu) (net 2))
 (segment (start 162.320002 87.63) (end 159.780002 85.09) (width 0.25) (layer B.Cu) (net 2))
 (segment (start 163.195 87.63) (end 162.320002 87.63) (width 0.25) (layer B.Cu) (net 2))
 (segment (start 159.780002 85.09) (end 154.305 85.09) (width 0.25) (layer B.Cu) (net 2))
 (segment (start 147.32 78.105) (end 147.32 76.2) (width 0.25) (layer B.Cu) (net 2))
 (segment (start 154.305 85.09) (end 147.32 78.105) (width 0.25) (layer B.Cu) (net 2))
 (segment (start 147.32 70.485) (end 147.32 76.2) (width 0.25) (layer B.Cu) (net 2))
 (segment (start 148.095 70.485) (end 150.82 67.76) (width 0.25) (layer B.Cu) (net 2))
 (segment (start 147.32 70.485) (end 148.095 70.485) (width 0.25) (layer B.Cu) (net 2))
 (segment (start 150.82 67.76) (end 150.82 66.35) (width 0.25) (layer B.Cu) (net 2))
 (segment (start 165.735 64.77) (end 165.735 54.61) (width 0.25) (layer B.Cu) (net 2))
 (segment (start 164.14 54.285) (end 162.56 52.705) (width 0.25) (layer B.Cu) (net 2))
 (segment (start 165.735 54.61) (end 165.41 54.285) (width 0.25) (layer B.Cu) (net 2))
 (segment (start 165.41 54.285) (end 164.14 54.285) (width 0.25) (layer B.Cu) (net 2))
 (segment (start 160.98 66.35) (end 162.56 64.77) (width 0.25) (layer B.Cu) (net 2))
 (segment (start 150.82 66.35) (end 160.98 66.35) (width 0.25) (layer B.Cu) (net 2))
 (segment (start 162.56 64.77) (end 165.735 64.77) (width 0.25) (layer B.Cu) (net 2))
 (segment (start 147.32 71.485) (end 147.32 70.485) (width 0.25) (layer B.Cu) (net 2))
 (segment (start 141.605 73.025) (end 147.32 73.025) (width 0.25) (layer B.Cu) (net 2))
 (segment (start 139.7 70.485) (end 139.7 71.485) (width 0.25) (layer B.Cu) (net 2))
 (segment (start 147.32 73.025) (end 147.32 71.485) (width 0.25) (layer B.Cu) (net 2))
 (segment (start 139.7 71.485) (end 141.605 73.025) (width 0.25) (layer B.Cu) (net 2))
 (segment (start 134.53 75.634315) (end 137.139315 73.025) (width 0.25) (layer F.Cu) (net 2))
 (segment (start 134.53 76.2) (end 134.53 75.634315) (width 0.25) (layer F.Cu) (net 2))
 (segment (start 138.43 73.025) (end 139.7 71.755) (width 0.25) (layer F.Cu) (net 2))
 (segment (start 139.7 76.835) (end 139.7 71.755) (width 0.25) (layer F.Cu) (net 2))
 (segment (start 137.139315 73.025) (end 138.43 73.025) (width 0.25) (layer F.Cu) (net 2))
 (segment (start 139.7 71.755) (end 139.7 70.485) (width 0.25) (layer F.Cu) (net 2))
 (segment (start 100.965 71.755) (end 100.965 78.105) (width 0.25) (layer F.Cu) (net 23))
 (segment (start 115.57 52.07) (end 115.57 57.15) (width 0.25) (layer F.Cu) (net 23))
 (segment (start 115.57 57.15) (end 100.965 71.755) (width 0.25) (layer F.Cu) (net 23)))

